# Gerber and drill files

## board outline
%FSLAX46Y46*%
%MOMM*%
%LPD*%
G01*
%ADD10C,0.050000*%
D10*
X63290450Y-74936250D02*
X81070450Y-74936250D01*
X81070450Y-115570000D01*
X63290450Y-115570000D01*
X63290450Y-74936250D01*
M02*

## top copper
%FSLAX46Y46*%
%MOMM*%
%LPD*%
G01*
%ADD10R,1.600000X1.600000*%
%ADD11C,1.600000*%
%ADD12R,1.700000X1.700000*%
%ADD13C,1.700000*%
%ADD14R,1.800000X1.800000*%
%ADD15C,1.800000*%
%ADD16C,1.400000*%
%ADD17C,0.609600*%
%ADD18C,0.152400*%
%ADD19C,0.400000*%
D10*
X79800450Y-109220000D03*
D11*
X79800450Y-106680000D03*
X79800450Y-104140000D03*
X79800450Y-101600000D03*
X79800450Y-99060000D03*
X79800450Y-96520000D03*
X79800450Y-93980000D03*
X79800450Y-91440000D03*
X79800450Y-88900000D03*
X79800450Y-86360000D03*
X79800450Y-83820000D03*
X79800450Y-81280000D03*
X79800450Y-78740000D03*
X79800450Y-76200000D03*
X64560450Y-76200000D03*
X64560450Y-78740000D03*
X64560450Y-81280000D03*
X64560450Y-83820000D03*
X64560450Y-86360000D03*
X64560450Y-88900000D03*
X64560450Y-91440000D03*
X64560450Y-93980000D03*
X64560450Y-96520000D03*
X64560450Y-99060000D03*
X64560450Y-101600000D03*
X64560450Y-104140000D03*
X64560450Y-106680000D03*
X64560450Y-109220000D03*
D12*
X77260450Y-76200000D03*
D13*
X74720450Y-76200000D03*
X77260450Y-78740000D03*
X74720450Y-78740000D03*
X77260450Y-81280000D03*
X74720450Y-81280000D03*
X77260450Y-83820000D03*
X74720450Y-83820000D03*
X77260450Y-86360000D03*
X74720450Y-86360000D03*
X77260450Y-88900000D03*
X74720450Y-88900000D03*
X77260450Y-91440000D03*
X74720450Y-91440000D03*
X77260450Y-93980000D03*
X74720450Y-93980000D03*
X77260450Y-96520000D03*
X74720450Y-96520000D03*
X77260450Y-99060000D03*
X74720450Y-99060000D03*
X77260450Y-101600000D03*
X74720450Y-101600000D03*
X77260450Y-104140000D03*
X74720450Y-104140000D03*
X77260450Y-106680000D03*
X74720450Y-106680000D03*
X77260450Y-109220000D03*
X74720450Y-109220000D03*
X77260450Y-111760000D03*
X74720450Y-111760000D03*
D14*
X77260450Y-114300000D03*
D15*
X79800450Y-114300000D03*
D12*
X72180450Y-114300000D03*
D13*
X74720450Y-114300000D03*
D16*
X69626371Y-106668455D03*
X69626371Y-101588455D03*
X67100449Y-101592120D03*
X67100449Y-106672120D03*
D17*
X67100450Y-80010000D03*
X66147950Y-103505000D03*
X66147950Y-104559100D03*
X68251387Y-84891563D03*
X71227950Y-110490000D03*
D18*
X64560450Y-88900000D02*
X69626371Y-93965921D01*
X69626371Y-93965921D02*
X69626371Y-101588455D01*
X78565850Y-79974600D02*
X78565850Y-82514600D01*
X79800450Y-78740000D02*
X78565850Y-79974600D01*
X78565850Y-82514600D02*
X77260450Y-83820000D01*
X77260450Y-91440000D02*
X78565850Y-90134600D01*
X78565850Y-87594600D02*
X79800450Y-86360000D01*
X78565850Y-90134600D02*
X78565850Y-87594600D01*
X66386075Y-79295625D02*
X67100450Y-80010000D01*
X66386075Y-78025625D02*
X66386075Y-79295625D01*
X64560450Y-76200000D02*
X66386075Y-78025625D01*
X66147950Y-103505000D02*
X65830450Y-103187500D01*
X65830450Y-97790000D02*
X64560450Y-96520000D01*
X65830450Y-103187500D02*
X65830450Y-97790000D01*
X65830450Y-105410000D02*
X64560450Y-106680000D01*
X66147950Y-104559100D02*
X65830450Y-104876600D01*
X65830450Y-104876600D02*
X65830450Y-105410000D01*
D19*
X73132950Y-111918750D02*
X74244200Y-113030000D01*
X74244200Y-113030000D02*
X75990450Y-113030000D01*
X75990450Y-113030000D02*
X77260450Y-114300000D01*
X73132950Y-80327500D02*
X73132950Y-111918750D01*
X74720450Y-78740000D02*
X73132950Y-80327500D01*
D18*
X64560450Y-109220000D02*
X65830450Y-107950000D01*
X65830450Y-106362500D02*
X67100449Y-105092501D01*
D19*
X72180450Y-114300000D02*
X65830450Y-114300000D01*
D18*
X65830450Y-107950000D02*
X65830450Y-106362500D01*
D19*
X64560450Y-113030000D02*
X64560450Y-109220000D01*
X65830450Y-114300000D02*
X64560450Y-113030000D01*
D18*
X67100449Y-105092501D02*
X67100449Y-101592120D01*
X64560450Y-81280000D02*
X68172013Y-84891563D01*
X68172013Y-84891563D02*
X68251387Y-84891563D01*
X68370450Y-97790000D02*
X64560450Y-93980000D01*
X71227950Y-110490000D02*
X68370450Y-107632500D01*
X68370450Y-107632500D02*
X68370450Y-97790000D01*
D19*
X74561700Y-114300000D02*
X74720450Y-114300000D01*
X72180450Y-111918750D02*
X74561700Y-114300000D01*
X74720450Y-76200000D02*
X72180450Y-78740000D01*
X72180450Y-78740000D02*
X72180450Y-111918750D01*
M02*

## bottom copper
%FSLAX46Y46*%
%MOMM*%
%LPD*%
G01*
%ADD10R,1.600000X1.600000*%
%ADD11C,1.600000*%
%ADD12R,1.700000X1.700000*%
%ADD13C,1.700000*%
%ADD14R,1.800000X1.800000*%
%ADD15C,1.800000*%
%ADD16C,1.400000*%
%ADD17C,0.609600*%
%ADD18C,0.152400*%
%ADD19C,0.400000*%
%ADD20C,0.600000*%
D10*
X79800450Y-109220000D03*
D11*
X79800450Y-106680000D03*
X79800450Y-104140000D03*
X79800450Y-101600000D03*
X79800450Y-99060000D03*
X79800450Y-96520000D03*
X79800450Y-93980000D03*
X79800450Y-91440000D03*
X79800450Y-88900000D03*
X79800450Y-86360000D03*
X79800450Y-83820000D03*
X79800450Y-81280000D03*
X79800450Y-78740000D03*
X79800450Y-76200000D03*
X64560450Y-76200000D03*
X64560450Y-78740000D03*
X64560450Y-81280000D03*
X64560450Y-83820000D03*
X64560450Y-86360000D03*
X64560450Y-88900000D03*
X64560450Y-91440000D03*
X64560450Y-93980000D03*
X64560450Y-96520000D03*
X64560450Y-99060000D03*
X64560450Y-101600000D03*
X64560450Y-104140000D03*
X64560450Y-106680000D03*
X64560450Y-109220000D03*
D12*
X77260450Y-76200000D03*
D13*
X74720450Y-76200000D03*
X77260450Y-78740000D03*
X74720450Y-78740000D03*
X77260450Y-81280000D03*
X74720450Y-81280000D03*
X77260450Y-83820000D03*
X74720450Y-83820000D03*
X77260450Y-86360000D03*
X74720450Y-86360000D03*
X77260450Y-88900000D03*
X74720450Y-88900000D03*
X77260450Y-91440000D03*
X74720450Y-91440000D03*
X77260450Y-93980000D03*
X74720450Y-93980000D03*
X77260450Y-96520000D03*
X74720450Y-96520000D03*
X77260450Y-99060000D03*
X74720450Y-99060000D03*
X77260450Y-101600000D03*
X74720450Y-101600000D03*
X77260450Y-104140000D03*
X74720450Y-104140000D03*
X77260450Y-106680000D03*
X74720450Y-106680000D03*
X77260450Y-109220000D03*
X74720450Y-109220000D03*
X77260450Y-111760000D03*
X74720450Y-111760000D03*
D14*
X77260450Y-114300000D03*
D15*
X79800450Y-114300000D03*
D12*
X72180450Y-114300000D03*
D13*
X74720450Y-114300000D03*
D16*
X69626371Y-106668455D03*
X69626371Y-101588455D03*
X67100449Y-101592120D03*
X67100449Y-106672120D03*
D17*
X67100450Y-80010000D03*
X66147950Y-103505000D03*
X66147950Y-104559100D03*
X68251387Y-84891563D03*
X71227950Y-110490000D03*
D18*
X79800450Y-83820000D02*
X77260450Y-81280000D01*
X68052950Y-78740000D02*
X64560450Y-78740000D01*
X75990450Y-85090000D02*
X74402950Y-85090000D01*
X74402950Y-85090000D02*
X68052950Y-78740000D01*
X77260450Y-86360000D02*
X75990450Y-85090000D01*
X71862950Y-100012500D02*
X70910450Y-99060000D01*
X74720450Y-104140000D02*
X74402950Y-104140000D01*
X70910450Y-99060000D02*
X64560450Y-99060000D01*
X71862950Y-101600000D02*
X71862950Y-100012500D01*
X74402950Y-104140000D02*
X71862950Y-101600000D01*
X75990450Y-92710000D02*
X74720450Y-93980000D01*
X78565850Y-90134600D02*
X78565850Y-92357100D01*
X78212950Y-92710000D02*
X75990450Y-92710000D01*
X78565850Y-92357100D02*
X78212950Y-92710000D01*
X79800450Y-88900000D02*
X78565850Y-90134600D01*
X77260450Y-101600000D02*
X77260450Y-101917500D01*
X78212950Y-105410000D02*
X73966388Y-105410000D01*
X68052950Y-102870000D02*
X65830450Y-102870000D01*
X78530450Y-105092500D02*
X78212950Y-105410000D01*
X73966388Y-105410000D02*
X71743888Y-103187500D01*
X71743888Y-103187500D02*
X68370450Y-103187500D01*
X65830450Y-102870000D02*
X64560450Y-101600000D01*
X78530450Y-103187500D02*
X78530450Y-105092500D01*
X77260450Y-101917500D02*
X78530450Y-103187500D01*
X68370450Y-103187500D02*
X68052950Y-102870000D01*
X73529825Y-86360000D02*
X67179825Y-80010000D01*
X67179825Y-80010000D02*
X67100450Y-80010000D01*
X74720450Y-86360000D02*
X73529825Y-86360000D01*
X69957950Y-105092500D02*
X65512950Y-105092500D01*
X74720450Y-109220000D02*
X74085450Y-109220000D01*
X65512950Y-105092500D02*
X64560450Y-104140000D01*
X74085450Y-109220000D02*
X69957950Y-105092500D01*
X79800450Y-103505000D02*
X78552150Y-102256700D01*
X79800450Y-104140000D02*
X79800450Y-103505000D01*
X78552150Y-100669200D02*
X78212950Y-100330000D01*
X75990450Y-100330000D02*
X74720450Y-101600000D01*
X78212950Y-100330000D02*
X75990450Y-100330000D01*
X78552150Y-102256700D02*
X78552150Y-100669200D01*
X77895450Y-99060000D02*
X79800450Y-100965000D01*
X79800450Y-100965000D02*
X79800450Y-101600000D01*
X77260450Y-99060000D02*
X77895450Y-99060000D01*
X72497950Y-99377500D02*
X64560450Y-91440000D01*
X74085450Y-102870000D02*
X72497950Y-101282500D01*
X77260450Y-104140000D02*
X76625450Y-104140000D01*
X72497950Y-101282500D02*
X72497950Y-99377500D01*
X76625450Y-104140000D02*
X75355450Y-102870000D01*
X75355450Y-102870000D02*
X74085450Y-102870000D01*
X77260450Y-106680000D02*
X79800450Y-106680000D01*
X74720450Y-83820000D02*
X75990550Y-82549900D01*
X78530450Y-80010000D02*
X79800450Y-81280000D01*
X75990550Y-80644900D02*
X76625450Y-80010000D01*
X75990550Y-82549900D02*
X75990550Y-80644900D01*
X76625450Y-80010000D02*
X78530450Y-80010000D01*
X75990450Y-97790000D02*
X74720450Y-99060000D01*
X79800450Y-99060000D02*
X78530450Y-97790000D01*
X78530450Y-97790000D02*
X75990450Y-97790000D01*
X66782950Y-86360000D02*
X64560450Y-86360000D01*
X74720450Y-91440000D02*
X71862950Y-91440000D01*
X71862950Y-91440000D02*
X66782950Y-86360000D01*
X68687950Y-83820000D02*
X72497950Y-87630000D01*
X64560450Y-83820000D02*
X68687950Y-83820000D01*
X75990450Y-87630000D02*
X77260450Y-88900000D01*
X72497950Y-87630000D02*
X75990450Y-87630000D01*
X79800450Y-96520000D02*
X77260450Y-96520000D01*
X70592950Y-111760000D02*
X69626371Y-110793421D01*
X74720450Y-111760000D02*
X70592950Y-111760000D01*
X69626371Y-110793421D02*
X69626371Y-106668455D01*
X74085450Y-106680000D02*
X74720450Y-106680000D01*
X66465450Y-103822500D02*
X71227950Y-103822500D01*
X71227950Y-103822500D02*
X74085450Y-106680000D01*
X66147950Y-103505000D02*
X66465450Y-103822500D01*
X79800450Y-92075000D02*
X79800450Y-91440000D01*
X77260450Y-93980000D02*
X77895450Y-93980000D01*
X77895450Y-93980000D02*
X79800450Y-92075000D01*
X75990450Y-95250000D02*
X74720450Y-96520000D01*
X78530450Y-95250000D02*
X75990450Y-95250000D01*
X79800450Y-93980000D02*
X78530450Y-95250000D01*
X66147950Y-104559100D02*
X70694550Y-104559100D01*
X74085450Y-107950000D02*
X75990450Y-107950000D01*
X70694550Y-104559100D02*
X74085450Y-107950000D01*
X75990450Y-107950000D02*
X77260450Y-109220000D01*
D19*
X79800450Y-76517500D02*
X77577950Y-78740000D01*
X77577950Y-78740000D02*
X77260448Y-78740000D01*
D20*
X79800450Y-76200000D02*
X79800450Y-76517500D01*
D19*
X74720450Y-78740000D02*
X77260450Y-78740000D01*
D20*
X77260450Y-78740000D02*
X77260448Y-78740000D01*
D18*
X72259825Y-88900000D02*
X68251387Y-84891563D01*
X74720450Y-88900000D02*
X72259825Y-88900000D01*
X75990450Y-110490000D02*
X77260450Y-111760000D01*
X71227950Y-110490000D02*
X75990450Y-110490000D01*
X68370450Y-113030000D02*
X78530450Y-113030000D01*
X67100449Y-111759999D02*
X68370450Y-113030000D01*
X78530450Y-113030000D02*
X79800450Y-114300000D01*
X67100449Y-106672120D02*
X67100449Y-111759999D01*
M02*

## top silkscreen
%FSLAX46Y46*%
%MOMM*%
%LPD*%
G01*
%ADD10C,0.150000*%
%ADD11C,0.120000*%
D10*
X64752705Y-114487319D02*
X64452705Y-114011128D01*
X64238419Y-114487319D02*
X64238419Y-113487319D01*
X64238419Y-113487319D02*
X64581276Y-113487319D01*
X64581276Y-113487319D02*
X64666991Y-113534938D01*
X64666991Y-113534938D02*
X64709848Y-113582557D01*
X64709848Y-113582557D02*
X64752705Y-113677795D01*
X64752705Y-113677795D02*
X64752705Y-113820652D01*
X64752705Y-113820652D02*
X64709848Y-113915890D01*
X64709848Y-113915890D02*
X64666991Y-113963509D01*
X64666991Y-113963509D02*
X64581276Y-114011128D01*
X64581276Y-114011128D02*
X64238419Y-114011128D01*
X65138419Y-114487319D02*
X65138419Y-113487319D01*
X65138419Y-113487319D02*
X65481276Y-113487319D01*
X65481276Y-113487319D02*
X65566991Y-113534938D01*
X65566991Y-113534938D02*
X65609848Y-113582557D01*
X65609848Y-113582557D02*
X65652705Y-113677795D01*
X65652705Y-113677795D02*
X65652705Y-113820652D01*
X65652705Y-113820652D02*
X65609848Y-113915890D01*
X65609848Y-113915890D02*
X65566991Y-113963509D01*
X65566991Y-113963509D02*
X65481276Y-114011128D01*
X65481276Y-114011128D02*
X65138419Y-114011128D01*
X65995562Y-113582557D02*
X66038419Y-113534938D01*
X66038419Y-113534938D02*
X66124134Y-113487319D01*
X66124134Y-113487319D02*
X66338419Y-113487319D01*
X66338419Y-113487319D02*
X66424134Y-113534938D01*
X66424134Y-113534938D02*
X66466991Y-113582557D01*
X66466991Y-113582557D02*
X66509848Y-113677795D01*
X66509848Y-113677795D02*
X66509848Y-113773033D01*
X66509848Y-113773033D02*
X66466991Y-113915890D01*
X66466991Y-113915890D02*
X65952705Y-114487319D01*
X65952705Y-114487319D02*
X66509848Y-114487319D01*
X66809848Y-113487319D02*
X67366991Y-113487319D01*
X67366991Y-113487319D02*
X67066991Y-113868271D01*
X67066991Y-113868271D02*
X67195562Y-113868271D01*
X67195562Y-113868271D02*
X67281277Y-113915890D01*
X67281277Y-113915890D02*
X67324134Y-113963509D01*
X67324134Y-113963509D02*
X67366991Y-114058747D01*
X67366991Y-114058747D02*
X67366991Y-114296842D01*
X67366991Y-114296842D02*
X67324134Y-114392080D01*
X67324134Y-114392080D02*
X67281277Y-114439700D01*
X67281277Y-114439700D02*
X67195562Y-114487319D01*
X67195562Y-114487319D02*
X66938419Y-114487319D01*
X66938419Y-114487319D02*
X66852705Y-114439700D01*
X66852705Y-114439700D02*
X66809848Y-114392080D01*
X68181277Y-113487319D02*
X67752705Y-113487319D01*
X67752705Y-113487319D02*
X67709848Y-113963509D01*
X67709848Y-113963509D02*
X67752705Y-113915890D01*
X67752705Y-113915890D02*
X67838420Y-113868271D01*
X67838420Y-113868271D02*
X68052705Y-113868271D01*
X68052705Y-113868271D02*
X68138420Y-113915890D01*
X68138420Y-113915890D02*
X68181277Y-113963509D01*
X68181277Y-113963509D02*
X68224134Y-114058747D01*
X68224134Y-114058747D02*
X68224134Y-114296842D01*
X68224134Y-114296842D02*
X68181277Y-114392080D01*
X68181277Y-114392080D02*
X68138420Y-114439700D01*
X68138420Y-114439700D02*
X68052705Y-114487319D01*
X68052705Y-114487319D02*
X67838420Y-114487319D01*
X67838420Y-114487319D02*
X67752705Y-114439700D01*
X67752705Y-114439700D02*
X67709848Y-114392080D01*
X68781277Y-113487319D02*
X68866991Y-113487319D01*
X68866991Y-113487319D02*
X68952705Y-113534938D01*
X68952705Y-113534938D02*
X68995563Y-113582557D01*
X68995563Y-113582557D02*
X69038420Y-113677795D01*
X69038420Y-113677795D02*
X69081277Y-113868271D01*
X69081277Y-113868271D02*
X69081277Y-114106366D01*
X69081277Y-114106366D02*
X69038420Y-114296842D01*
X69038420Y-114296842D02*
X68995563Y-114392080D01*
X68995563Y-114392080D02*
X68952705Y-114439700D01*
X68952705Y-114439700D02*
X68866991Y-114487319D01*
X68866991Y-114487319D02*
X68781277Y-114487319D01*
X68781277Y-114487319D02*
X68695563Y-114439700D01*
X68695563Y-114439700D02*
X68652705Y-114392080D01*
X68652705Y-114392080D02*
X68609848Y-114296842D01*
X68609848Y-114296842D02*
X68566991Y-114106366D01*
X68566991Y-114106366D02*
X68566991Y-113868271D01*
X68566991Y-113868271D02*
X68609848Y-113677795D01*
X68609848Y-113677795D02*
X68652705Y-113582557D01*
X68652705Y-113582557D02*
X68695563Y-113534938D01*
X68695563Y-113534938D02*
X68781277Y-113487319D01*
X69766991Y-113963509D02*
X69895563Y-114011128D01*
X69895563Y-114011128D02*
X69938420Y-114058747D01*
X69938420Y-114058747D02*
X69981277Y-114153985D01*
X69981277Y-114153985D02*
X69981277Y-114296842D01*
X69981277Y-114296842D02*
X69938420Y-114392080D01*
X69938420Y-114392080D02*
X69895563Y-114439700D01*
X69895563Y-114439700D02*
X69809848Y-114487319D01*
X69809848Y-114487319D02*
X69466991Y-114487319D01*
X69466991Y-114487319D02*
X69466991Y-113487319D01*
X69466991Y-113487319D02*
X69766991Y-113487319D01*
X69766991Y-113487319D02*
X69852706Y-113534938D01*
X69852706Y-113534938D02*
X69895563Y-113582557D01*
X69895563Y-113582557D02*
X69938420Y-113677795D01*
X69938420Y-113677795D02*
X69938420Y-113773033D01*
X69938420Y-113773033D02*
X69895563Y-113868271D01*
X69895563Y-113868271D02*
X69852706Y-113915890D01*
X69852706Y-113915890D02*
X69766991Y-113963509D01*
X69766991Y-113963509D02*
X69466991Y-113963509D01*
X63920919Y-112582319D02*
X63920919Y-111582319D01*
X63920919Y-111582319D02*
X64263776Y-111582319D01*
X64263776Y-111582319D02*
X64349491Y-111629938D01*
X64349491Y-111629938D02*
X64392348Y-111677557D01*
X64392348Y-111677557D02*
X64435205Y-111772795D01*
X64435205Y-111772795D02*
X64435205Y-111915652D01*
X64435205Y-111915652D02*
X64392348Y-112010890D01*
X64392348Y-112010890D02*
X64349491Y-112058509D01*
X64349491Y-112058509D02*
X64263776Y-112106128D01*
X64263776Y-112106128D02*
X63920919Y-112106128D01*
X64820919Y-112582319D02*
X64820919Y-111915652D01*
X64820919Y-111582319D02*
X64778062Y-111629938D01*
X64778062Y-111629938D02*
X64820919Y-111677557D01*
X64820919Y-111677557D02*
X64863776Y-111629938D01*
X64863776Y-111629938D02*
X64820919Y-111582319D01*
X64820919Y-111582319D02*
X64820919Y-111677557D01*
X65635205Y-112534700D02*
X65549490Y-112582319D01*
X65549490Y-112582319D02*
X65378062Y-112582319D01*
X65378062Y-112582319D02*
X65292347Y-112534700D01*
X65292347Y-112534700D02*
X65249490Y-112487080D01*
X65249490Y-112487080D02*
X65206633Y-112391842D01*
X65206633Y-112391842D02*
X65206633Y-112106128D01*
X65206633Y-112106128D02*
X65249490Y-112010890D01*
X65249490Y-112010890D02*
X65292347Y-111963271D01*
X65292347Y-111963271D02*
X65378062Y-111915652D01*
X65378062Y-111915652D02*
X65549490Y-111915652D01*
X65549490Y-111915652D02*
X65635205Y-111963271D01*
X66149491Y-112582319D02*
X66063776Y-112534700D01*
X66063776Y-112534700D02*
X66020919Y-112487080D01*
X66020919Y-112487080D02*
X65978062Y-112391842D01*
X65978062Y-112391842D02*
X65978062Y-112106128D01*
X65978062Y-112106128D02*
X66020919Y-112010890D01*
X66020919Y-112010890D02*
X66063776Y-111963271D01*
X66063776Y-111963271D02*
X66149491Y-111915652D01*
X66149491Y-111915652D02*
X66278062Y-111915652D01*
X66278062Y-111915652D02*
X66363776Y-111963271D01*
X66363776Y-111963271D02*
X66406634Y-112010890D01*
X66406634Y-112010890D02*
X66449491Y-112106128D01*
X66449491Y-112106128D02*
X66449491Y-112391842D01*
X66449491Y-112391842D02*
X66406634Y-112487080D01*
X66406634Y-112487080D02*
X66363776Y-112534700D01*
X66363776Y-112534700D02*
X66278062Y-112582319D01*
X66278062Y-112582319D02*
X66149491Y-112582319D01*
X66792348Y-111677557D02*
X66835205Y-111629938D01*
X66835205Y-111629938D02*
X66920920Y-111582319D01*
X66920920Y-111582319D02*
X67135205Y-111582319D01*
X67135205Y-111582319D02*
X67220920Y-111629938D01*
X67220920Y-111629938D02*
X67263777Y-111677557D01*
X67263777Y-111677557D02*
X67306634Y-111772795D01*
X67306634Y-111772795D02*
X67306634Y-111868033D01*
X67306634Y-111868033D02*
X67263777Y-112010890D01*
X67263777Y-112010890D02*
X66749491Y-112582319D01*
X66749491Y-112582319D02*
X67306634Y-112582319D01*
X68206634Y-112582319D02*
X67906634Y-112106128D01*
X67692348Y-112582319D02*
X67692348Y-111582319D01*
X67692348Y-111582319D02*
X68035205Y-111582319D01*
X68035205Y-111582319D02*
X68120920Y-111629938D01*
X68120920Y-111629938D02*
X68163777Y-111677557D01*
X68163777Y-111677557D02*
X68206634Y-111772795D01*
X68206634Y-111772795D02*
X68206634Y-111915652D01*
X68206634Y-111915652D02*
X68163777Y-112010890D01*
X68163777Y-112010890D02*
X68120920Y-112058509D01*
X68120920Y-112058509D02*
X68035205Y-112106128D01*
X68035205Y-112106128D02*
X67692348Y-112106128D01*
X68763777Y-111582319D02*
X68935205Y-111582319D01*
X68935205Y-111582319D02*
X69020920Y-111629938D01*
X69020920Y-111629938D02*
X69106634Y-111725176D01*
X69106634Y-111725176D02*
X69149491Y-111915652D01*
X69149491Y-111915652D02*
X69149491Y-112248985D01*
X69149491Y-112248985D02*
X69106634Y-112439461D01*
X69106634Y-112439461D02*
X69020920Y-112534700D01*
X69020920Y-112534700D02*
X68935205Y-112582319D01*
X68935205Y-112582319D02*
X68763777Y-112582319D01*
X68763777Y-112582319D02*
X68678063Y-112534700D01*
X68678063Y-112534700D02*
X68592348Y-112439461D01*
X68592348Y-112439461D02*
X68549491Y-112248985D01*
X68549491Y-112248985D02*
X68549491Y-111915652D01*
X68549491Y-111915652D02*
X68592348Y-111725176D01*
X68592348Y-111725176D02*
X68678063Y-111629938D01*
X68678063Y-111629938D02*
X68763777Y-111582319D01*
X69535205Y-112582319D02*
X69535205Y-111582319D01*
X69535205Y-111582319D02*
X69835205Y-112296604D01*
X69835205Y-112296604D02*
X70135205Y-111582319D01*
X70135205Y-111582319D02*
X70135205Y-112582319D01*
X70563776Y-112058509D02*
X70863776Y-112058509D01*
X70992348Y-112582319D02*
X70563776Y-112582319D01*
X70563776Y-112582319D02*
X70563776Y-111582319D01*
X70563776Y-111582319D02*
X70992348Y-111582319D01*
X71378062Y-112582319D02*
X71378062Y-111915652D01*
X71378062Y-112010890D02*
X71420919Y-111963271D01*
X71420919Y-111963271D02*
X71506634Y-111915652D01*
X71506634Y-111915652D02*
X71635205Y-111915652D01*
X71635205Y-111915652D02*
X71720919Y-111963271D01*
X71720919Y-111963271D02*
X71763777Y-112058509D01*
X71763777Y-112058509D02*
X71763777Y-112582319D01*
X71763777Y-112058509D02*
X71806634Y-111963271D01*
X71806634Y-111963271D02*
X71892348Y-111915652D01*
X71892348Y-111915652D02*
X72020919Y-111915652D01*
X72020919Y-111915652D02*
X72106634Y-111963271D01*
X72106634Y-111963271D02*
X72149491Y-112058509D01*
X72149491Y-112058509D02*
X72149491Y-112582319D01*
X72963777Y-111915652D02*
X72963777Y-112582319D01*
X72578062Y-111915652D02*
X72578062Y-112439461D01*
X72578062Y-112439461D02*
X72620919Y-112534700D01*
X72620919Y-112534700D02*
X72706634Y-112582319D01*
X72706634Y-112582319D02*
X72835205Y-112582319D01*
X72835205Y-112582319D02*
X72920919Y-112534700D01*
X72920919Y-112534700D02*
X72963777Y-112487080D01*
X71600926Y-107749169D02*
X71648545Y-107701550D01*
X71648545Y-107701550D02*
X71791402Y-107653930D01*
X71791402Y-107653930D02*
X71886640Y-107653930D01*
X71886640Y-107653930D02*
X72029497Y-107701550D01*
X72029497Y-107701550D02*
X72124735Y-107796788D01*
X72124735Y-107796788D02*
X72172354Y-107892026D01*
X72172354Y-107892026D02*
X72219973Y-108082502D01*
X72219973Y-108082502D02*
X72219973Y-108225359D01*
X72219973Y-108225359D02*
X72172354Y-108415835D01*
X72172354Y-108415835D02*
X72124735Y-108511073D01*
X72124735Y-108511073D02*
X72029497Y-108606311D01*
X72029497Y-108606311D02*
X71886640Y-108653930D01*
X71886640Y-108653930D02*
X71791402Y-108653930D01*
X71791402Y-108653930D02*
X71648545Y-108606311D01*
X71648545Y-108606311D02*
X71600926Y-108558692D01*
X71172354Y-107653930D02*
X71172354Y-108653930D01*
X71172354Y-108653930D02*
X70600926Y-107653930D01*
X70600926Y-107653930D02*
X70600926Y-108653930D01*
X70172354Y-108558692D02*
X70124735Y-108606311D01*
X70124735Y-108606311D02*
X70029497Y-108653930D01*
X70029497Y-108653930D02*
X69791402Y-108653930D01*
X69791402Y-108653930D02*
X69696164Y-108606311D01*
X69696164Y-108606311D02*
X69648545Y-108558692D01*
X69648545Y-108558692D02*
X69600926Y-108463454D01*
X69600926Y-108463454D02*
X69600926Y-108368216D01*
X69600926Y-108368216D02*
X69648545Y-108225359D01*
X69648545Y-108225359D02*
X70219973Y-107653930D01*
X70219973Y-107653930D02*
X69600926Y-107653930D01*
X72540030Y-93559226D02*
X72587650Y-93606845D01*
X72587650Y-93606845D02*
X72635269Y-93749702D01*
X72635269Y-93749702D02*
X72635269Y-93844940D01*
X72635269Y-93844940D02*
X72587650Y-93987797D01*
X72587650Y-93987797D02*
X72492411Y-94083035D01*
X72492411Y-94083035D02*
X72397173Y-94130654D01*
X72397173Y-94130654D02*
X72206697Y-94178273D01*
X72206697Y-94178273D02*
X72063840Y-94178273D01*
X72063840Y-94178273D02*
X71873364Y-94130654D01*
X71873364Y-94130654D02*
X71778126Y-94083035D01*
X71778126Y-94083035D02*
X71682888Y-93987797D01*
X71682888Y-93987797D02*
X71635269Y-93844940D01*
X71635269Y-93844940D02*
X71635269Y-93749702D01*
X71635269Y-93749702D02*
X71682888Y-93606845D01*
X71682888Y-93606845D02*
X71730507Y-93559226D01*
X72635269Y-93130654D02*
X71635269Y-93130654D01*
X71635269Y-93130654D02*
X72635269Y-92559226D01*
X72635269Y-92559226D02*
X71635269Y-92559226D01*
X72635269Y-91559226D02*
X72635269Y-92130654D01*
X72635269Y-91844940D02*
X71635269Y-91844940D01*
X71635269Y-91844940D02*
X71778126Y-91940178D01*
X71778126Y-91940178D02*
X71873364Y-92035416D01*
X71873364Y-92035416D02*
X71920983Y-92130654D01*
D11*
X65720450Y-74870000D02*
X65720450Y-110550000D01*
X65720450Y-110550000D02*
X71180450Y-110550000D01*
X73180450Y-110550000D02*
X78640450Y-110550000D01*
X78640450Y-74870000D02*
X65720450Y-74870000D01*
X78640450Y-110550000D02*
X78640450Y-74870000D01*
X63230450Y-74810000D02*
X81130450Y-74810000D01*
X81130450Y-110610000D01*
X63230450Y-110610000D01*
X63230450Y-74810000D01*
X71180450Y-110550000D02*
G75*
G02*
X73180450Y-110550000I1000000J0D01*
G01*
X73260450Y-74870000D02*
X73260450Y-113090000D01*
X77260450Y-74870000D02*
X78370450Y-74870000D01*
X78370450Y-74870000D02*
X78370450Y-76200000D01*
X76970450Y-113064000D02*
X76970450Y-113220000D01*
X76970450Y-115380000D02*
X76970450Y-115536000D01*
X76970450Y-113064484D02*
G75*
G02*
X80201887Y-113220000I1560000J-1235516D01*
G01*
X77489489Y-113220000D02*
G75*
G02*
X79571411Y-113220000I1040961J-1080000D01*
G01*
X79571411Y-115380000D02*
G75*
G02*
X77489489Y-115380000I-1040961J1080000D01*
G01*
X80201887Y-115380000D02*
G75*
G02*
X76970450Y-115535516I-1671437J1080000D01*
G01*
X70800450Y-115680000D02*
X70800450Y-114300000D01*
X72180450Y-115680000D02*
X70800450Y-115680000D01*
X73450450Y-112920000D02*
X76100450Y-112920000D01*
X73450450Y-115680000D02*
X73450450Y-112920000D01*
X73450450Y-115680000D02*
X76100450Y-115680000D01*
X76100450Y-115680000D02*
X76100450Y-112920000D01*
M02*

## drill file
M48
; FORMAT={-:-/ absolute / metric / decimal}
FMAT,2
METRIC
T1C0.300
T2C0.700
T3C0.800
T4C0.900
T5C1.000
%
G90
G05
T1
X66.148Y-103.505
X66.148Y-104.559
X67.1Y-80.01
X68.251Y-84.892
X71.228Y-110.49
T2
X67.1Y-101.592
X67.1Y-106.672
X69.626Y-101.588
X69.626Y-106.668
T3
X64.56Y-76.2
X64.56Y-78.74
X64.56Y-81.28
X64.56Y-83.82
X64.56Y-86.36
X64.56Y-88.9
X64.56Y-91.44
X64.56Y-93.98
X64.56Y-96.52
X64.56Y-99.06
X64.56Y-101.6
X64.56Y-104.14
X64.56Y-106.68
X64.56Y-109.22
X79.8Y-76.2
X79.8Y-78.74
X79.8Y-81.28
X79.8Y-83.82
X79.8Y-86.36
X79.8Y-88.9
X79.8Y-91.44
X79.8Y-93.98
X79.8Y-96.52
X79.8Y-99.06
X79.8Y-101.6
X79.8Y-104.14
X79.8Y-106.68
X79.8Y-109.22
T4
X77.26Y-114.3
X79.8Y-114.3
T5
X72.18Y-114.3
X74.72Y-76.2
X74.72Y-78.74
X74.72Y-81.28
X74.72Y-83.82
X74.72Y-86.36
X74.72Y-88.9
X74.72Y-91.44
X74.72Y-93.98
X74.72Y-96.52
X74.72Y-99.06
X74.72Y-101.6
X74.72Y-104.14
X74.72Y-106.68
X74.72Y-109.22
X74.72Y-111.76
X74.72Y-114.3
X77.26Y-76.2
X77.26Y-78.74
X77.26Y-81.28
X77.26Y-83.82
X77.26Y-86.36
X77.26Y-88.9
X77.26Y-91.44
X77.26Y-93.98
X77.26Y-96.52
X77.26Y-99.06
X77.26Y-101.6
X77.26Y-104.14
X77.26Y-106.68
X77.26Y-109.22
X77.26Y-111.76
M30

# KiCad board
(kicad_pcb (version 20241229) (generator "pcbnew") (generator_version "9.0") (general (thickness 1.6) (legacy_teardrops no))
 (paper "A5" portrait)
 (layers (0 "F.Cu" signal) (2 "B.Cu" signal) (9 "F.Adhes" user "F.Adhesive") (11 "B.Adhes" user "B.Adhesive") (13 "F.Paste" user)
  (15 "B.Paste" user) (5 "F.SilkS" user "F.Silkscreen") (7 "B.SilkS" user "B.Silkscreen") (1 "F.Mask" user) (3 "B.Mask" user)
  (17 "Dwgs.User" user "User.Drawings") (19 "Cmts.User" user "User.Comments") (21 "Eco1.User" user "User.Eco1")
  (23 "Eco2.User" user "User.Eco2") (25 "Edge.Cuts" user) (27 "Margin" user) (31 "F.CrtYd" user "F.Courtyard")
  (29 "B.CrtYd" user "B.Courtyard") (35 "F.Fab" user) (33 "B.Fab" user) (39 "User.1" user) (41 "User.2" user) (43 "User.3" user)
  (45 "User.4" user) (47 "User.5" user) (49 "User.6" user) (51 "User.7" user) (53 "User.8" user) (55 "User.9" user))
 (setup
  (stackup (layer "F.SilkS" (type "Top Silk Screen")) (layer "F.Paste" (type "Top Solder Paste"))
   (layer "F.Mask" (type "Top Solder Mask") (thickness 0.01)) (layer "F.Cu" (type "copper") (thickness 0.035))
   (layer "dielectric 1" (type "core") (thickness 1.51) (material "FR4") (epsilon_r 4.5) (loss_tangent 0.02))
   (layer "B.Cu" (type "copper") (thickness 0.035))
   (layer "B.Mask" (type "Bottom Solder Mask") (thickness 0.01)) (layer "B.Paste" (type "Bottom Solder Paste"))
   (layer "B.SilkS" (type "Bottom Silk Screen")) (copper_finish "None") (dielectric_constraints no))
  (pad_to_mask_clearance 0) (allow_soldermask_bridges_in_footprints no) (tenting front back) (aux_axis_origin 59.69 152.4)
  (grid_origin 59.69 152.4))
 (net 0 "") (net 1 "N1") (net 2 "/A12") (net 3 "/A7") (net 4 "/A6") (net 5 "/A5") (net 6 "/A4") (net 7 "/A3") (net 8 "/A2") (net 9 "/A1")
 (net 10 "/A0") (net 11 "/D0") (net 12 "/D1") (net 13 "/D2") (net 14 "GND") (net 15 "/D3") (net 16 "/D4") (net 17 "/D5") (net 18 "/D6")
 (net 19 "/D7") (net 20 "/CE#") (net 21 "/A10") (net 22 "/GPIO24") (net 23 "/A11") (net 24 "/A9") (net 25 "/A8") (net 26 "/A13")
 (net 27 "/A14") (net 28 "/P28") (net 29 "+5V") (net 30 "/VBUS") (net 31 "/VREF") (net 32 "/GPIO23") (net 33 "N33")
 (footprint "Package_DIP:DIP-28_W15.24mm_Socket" (layer "F.Cu") (at 79.80045 109.22 180)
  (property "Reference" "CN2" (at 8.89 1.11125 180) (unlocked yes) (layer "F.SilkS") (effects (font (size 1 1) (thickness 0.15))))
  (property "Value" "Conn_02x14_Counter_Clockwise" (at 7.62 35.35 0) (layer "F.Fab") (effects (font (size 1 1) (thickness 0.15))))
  (fp_line (start 14.08 34.35) (end 14.08 -1.33) (stroke (width 0.12) (type solid)) (layer "F.SilkS"))
  (fp_line (start 14.08 -1.33) (end 8.62 -1.33) (stroke (width 0.12) (type solid)) (layer "F.SilkS"))
  (fp_line (start 6.62 -1.33) (end 1.16 -1.33) (stroke (width 0.12) (type solid)) (layer "F.SilkS"))
  (fp_line (start 1.16 34.35) (end 14.08 34.35) (stroke (width 0.12) (type solid)) (layer "F.SilkS"))
  (fp_line (start 1.16 -1.33) (end 1.16 34.35) (stroke (width 0.12) (type solid)) (layer "F.SilkS"))
  (fp_rect (start -1.33 -1.39) (end 16.57 34.41) (stroke (width 0.12) (type solid)) (fill no) (layer "F.SilkS"))
  (fp_arc (start 8.62 -1.33) (mid 7.62 -0.33) (end 6.62 -1.33) (stroke (width 0.12) (type solid)) (layer "F.SilkS"))
  (pad "1" thru_hole rect (at 0 0 180) (size 1.6 1.6) (drill 0.8) (layers "*.Cu" "*.Mask") (remove_unused_layers no) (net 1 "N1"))
  (pad "2" thru_hole circle (at 0 2.54 180) (size 1.6 1.6) (drill 0.8) (layers "*.Cu" "*.Mask") (remove_unused_layers no) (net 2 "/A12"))
  (pad "3" thru_hole circle (at 0 5.08 180) (size 1.6 1.6) (drill 0.8) (layers "*.Cu" "*.Mask") (remove_unused_layers no) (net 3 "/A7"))
  (pad "4" thru_hole circle (at 0 7.62 180) (size 1.6 1.6) (drill 0.8) (layers "*.Cu" "*.Mask") (remove_unused_layers no) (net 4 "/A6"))
  (pad "5" thru_hole circle (at 0 10.16 180) (size 1.6 1.6) (drill 0.8) (layers "*.Cu" "*.Mask") (remove_unused_layers no) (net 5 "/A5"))
  (pad "6" thru_hole circle (at 0 12.7 180) (size 1.6 1.6) (drill 0.8) (layers "*.Cu" "*.Mask") (remove_unused_layers no) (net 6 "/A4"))
  (pad "7" thru_hole circle (at 0 15.24 180) (size 1.6 1.6) (drill 0.8) (layers "*.Cu" "*.Mask") (remove_unused_layers no) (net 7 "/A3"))
  (pad "8" thru_hole circle (at 0 17.78 180) (size 1.6 1.6) (drill 0.8) (layers "*.Cu" "*.Mask") (remove_unused_layers no) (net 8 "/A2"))
  (pad "9" thru_hole circle (at 0 20.32 180) (size 1.6 1.6) (drill 0.8) (layers "*.Cu" "*.Mask") (remove_unused_layers no) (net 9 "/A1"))
  (pad "10" thru_hole circle (at 0 22.86 180) (size 1.6 1.6) (drill 0.8) (layers "*.Cu" "*.Mask") (remove_unused_layers no) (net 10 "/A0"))
  (pad "11" thru_hole circle (at 0 25.4 180) (size 1.6 1.6) (drill 0.8) (layers "*.Cu" "*.Mask") (remove_unused_layers no) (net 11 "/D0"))
  (pad "12" thru_hole circle (at 0 27.94 180) (size 1.6 1.6) (drill 0.8) (layers "*.Cu" "*.Mask") (remove_unused_layers no) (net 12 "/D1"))
  (pad "13" thru_hole circle (at 0 30.48 180) (size 1.6 1.6) (drill 0.8) (layers "*.Cu" "*.Mask") (remove_unused_layers no) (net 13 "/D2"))
  (pad "14" thru_hole circle (at 0 33.02 180) (size 1.6 1.6) (drill 0.8) (layers "*.Cu" "*.Mask") (remove_unused_layers no) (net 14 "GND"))
  (pad "15" thru_hole circle (at 15.24 33.02 180) (size 1.6 1.6) (drill 0.8) (layers "*.Cu" "*.Mask") (remove_unused_layers no)
   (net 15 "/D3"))
  (pad "16" thru_hole circle (at 15.24 30.48 180) (size 1.6 1.6) (drill 0.8) (layers "*.Cu" "*.Mask") (remove_unused_layers no)
   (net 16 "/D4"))
  (pad "17" thru_hole circle (at 15.24 27.94 180) (size 1.6 1.6) (drill 0.8) (layers "*.Cu" "*.Mask") (remove_unused_layers no)
   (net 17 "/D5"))
  (pad "18" thru_hole circle (at 15.24 25.4 180) (size 1.6 1.6) (drill 0.8) (layers "*.Cu" "*.Mask") (remove_unused_layers no)
   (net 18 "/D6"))
  (pad "19" thru_hole circle (at 15.24 22.86 180) (size 1.6 1.6) (drill 0.8) (layers "*.Cu" "*.Mask") (remove_unused_layers no)
   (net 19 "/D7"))
  (pad "20" thru_hole circle (at 15.24 20.32 180) (size 1.6 1.6) (drill 0.8) (layers "*.Cu" "*.Mask") (remove_unused_layers no)
   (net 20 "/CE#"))
  (pad "21" thru_hole circle (at 15.24 17.78 180) (size 1.6 1.6) (drill 0.8) (layers "*.Cu" "*.Mask") (remove_unused_layers no)
   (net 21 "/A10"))
  (pad "22" thru_hole circle (at 15.24 15.24 180) (size 1.6 1.6) (drill 0.8) (layers "*.Cu" "*.Mask") (remove_unused_layers no)
   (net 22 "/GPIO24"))
  (pad "23" thru_hole circle (at 15.24 12.7 180) (size 1.6 1.6) (drill 0.8) (layers "*.Cu" "*.Mask") (remove_unused_layers no)
   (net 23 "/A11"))
  (pad "24" thru_hole circle (at 15.24 10.16 180) (size 1.6 1.6) (drill 0.8) (layers "*.Cu" "*.Mask") (remove_unused_layers no)
   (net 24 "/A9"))
  (pad "25" thru_hole circle (at 15.24 7.62 180) (size 1.6 1.6) (drill 0.8) (layers "*.Cu" "*.Mask") (remove_unused_layers no)
   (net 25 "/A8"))
  (pad "26" thru_hole circle (at 15.24 5.08 180) (size 1.6 1.6) (drill 0.8) (layers "*.Cu" "*.Mask") (remove_unused_layers no)
   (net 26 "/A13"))
  (pad "27" thru_hole circle (at 15.24 2.54 180) (size 1.6 1.6) (drill 0.8) (layers "*.Cu" "*.Mask") (remove_unused_layers no)
   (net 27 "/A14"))
  (pad "28" thru_hole circle (at 15.24 0 180) (size 1.6 1.6) (drill 0.8) (layers "*.Cu" "*.Mask") (remove_unused_layers no) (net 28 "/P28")))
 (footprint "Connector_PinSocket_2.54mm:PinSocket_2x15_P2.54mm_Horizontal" (layer "F.Cu") (at 77.26045 76.2)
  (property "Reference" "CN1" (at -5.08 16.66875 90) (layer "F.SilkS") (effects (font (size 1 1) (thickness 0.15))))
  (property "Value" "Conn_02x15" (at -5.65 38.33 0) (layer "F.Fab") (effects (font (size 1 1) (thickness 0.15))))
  (fp_line (start -4 -1.33) (end -4 36.89) (stroke (width 0.12) (type solid)) (layer "F.SilkS"))
  (fp_line (start 0 -1.33) (end 1.11 -1.33) (stroke (width 0.12) (type solid)) (layer "F.SilkS"))
  (fp_line (start 1.11 -1.33) (end 1.11 0) (stroke (width 0.12) (type solid)) (layer "F.SilkS"))
  (pad "1" thru_hole rect (at 0 0) (size 1.7 1.7) (drill 1) (layers "*.Cu" "*.Mask") (remove_unused_layers no) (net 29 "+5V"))
  (pad "2" thru_hole circle (at -2.54 0) (size 1.7 1.7) (drill 1) (layers "*.Cu" "*.Mask") (remove_unused_layers no) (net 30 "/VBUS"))
  (pad "3" thru_hole circle (at 0 2.54) (size 1.7 1.7) (drill 1) (layers "*.Cu" "*.Mask") (remove_unused_layers no) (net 14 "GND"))
  (pad "4" thru_hole circle (at -2.54 2.54) (size 1.7 1.7) (drill 1) (layers "*.Cu" "*.Mask") (remove_unused_layers no) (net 14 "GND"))
  (pad "5" thru_hole circle (at 0 5.08) (size 1.7 1.7) (drill 1) (layers "*.Cu" "*.Mask") (remove_unused_layers no) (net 11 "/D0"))
  (pad "6" thru_hole circle (at -2.54 5.08) (size 1.7 1.7) (drill 1) (layers "*.Cu" "*.Mask") (remove_unused_layers no) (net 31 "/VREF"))
  (pad "7" thru_hole circle (at 0 7.62) (size 1.7 1.7) (drill 1) (layers "*.Cu" "*.Mask") (remove_unused_layers no) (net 13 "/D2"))
  (pad "8" thru_hole circle (at -2.54 7.62) (size 1.7 1.7) (drill 1) (layers "*.Cu" "*.Mask") (remove_unused_layers no) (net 12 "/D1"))
  (pad "9" thru_hole circle (at 0 10.16) (size 1.7 1.7) (drill 1) (layers "*.Cu" "*.Mask") (remove_unused_layers no) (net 16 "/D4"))
  (pad "10" thru_hole circle (at -2.54 10.16) (size 1.7 1.7) (drill 1) (layers "*.Cu" "*.Mask") (remove_unused_layers no) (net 15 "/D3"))
  (pad "11" thru_hole circle (at 0 12.7) (size 1.7 1.7) (drill 1) (layers "*.Cu" "*.Mask") (remove_unused_layers no) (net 18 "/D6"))
  (pad "12" thru_hole circle (at -2.54 12.7) (size 1.7 1.7) (drill 1) (layers "*.Cu" "*.Mask") (remove_unused_layers no) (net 17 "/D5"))
  (pad "13" thru_hole circle (at 0 15.24) (size 1.7 1.7) (drill 1) (layers "*.Cu" "*.Mask") (remove_unused_layers no) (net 10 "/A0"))
  (pad "14" thru_hole circle (at -2.54 15.24) (size 1.7 1.7) (drill 1) (layers "*.Cu" "*.Mask") (remove_unused_layers no) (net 19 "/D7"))
  (pad "15" thru_hole circle (at 0 17.78) (size 1.7 1.7) (drill 1) (layers "*.Cu" "*.Mask") (remove_unused_layers no) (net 8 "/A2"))
  (pad "16" thru_hole circle (at -2.54 17.78) (size 1.7 1.7) (drill 1) (layers "*.Cu" "*.Mask") (remove_unused_layers no) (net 9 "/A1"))
  (pad "17" thru_hole circle (at 0 20.32) (size 1.7 1.7) (drill 1) (layers "*.Cu" "*.Mask") (remove_unused_layers no) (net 6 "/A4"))
  (pad "18" thru_hole circle (at -2.54 20.32) (size 1.7 1.7) (drill 1) (layers "*.Cu" "*.Mask") (remove_unused_layers no) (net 7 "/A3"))
  (pad "19" thru_hole circle (at 0 22.86) (size 1.7 1.7) (drill 1) (layers "*.Cu" "*.Mask") (remove_unused_layers no) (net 4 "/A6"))
  (pad "20" thru_hole circle (at -2.54 22.86) (size 1.7 1.7) (drill 1) (layers "*.Cu" "*.Mask") (remove_unused_layers no) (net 5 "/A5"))
  (pad "21" thru_hole circle (at 0 25.4) (size 1.7 1.7) (drill 1) (layers "*.Cu" "*.Mask") (remove_unused_layers no) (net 25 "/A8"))
  (pad "22" thru_hole circle (at -2.54 25.4) (size 1.7 1.7) (drill 1) (layers "*.Cu" "*.Mask") (remove_unused_layers no) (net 3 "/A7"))
  (pad "23" thru_hole circle (at 0 27.94) (size 1.7 1.7) (drill 1) (layers "*.Cu" "*.Mask") (remove_unused_layers no) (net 21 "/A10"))
  (pad "24" thru_hole circle (at -2.54 27.94) (size 1.7 1.7) (drill 1) (layers "*.Cu" "*.Mask") (remove_unused_layers no) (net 24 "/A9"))
  (pad "25" thru_hole circle (at 0 30.48) (size 1.7 1.7) (drill 1) (layers "*.Cu" "*.Mask") (remove_unused_layers no) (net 2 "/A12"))
  (pad "26" thru_hole circle (at -2.54 30.48) (size 1.7 1.7) (drill 1) (layers "*.Cu" "*.Mask") (remove_unused_layers no) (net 23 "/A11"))
  (pad "27" thru_hole circle (at 0 33.02) (size 1.7 1.7) (drill 1) (layers "*.Cu" "*.Mask") (remove_unused_layers no) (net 27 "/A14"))
  (pad "28" thru_hole circle (at -2.54 33.02) (size 1.7 1.7) (drill 1) (layers "*.Cu" "*.Mask") (remove_unused_layers no) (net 26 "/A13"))
  (pad "29" thru_hole circle (at 0 35.56) (size 1.7 1.7) (drill 1) (layers "*.Cu" "*.Mask") (remove_unused_layers no) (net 22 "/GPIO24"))
  (pad "30" thru_hole circle (at -2.54 35.56) (size 1.7 1.7) (drill 1) (layers "*.Cu" "*.Mask") (remove_unused_layers no) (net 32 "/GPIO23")))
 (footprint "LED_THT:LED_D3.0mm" (layer "F.Cu") (at 77.26045 114.3)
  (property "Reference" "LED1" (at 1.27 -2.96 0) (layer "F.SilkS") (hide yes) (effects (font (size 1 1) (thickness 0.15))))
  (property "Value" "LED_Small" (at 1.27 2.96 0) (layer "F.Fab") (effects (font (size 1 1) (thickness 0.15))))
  (fp_line (start -0.29 -1.236) (end -0.29 -1.08) (stroke (width 0.12) (type solid)) (layer "F.SilkS"))
  (fp_line (start -0.29 1.08) (end -0.29 1.236) (stroke (width 0.12) (type solid)) (layer "F.SilkS"))
  (fp_arc (start -0.29 -1.235516) (mid 1.36566 -1.987699) (end 2.941437 -1.08) (stroke (width 0.12) (type solid)) (layer "F.SilkS"))
  (fp_arc (start 0.229039 -1.08) (mid 1.27 -1.5) (end 2.310961 -1.08) (stroke (width 0.12) (type solid)) (layer "F.SilkS"))
  (fp_arc (start 2.310961 1.08) (mid 1.27 1.5) (end 0.229039 1.08) (stroke (width 0.12) (type solid)) (layer "F.SilkS"))
  (fp_arc (start 2.941437 1.08) (mid 1.36566 1.987699) (end -0.29 1.235516) (stroke (width 0.12) (type solid)) (layer "F.SilkS"))
  (pad "1" thru_hole rect (at 0 0) (size 1.8 1.8) (drill 0.9) (layers "*.Cu" "*.Mask") (remove_unused_layers no) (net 14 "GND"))
  (pad "2" thru_hole circle (at 2.54 0) (size 1.8 1.8) (drill 0.9) (layers "*.Cu" "*.Mask") (remove_unused_layers no) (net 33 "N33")))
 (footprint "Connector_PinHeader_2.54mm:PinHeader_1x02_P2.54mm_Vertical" (layer "F.Cu") (at 72.18045 114.3 90)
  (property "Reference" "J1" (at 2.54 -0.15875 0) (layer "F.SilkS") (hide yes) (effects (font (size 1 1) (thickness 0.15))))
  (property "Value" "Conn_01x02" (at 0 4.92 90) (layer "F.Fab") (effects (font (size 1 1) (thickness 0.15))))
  (fp_line (start -1.38 -1.38) (end 0 -1.38) (stroke (width 0.12) (type solid)) (layer "F.SilkS"))
  (fp_line (start -1.38 0) (end -1.38 -1.38) (stroke (width 0.12) (type solid)) (layer "F.SilkS"))
  (fp_line (start 1.38 1.27) (end 1.38 3.92) (stroke (width 0.12) (type solid)) (layer "F.SilkS"))
  (fp_line (start -1.38 1.27) (end 1.38 1.27) (stroke (width 0.12) (type solid)) (layer "F.SilkS"))
  (fp_line (start -1.38 1.27) (end -1.38 3.92) (stroke (width 0.12) (type solid)) (layer "F.SilkS"))
  (fp_line (start -1.38 3.92) (end 1.38 3.92) (stroke (width 0.12) (type solid)) (layer "F.SilkS"))
  (pad "1" thru_hole rect (at 0 0 90) (size 1.7 1.7) (drill 1) (layers "*.Cu" "*.Mask") (remove_unused_layers no) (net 28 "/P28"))
  (pad "2" thru_hole circle (at 0 2.54 90) (size 1.7 1.7) (drill 1) (layers "*.Cu" "*.Mask") (remove_unused_layers no) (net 30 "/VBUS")))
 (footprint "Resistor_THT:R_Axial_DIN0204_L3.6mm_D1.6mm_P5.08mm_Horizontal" (layer "B.Cu") (at 69.626371 106.668455 90)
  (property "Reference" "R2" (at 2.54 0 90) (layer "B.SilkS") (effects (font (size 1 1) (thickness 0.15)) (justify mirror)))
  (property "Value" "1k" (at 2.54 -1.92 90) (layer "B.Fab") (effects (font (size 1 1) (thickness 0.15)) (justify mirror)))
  (pad "1" thru_hole circle (at 0 0 90) (size 1.4 1.4) (drill 0.7) (layers "*.Cu" "*.Mask") (remove_unused_layers no) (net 32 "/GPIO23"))
  (pad "2" thru_hole circle (at 5.08 0 90) (size 1.4 1.4) (drill 0.7) (layers "*.Cu" "*.Mask") (remove_unused_layers no) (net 20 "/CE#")))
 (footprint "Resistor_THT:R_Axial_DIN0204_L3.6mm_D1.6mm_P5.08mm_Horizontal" (layer "B.Cu") (at 67.100449 101.59212 -90)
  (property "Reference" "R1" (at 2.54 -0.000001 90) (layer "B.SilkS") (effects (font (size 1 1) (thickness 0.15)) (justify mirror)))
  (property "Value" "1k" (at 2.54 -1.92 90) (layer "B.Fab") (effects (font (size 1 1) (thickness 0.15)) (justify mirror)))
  (pad "1" thru_hole circle (at 0 0 270) (size 1.4 1.4) (drill 0.7) (layers "*.Cu" "*.Mask") (remove_unused_layers no) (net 28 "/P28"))
  (pad "2" thru_hole circle (at 5.08 0 270) (size 1.4 1.4) (drill 0.7) (layers "*.Cu" "*.Mask") (remove_unused_layers no) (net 33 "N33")))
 (gr_rect (start 63.29045 74.93625) (end 81.07045 115.57) (stroke (width 0.05) (type default)) (fill no) (layer "Edge.Cuts"))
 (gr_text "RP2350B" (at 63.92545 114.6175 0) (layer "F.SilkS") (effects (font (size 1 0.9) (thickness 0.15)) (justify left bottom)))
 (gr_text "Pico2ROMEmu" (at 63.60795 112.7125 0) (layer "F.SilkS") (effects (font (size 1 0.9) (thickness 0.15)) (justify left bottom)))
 (segment (start 64.56045 88.9) (end 69.626371 93.965921) (width 0.1524) (layer "F.Cu") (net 20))
 (segment (start 69.626371 93.965921) (end 69.626371 101.588455) (width 0.1524) (layer "F.Cu") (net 20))
 (segment (start 79.80045 83.82) (end 77.26045 81.28) (width 0.1524) (layer "B.Cu") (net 11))
 (segment (start 68.05295 78.74) (end 64.56045 78.74) (width 0.1524) (layer "B.Cu") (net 16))
 (segment (start 75.99045 85.09) (end 74.40295 85.09) (width 0.1524) (layer "B.Cu") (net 16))
 (segment (start 74.40295 85.09) (end 68.05295 78.74) (width 0.1524) (layer "B.Cu") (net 16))
 (segment (start 77.26045 86.36) (end 75.99045 85.09) (width 0.1524) (layer "B.Cu") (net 16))
 (segment (start 71.86295 100.0125) (end 70.91045 99.06) (width 0.1524) (layer "B.Cu") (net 24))
 (segment (start 74.72045 104.14) (end 74.40295 104.14) (width 0.1524) (layer "B.Cu") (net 24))
 (segment (start 70.91045 99.06) (end 64.56045 99.06) (width 0.1524) (layer "B.Cu") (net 24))
 (segment (start 71.86295 101.6) (end 71.86295 100.0125) (width 0.1524) (layer "B.Cu") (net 24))
 (segment (start 74.40295 104.14) (end 71.86295 101.6) (width 0.1524) (layer "B.Cu") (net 24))
 (segment (start 78.56585 79.9746) (end 78.56585 82.5146) (width 0.1524) (layer "F.Cu") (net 13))
 (segment (start 79.80045 78.74) (end 78.56585 79.9746) (width 0.1524) (layer "F.Cu") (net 13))
 (segment (start 78.56585 82.5146) (end 77.26045 83.82) (width 0.1524) (layer "F.Cu") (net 13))
 (segment (start 75.99045 92.71) (end 74.72045 93.98) (width 0.1524) (layer "B.Cu") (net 9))
 (segment (start 78.56585 90.1346) (end 78.56585 92.3571) (width 0.1524) (layer "B.Cu") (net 9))
 (segment (start 78.21295 92.71) (end 75.99045 92.71) (width 0.1524) (layer "B.Cu") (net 9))
 (segment (start 78.56585 92.3571) (end 78.21295 92.71) (width 0.1524) (layer "B.Cu") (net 9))
 (segment (start 79.80045 88.9) (end 78.56585 90.1346) (width 0.1524) (layer "B.Cu") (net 9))
 (segment (start 77.26045 101.6) (end 77.26045 101.9175) (width 0.1524) (layer "B.Cu") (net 25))
 (segment (start 78.21295 105.41) (end 73.966388 105.41) (width 0.1524) (layer "B.Cu") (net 25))
 (segment (start 68.05295 102.87) (end 65.83045 102.87) (width 0.1524) (layer "B.Cu") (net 25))
 (segment (start 78.53045 105.0925) (end 78.21295 105.41) (width 0.1524) (layer "B.Cu") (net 25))
 (segment (start 73.966388 105.41) (end 71.743888 103.1875) (width 0.1524) (layer "B.Cu") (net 25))
 (segment (start 71.743888 103.1875) (end 68.37045 103.1875) (width 0.1524) (layer "B.Cu") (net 25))
 (segment (start 65.83045 102.87) (end 64.56045 101.6) (width 0.1524) (layer "B.Cu") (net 25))
 (segment (start 78.53045 103.1875) (end 78.53045 105.0925) (width 0.1524) (layer "B.Cu") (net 25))
 (segment (start 77.26045 101.9175) (end 78.53045 103.1875) (width 0.1524) (layer "B.Cu") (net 25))
 (segment (start 68.37045 103.1875) (end 68.05295 102.87) (width 0.1524) (layer "B.Cu") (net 25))
 (segment (start 77.26045 91.44) (end 78.56585 90.1346) (width 0.1524) (layer "F.Cu") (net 10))
 (segment (start 78.56585 87.5946) (end 79.80045 86.36) (width 0.1524) (layer "F.Cu") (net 10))
 (segment (start 78.56585 90.1346) (end 78.56585 87.5946) (width 0.1524) (layer "F.Cu") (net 10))
 (segment (start 66.386075 79.295625) (end 67.10045 80.01) (width 0.1524) (layer "F.Cu") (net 15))
 (segment (start 66.386075 78.025625) (end 66.386075 79.295625) (width 0.1524) (layer "F.Cu") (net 15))
 (segment (start 64.56045 76.2) (end 66.386075 78.025625) (width 0.1524) (layer "F.Cu") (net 15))
 (via (at 67.10045 80.01) (size 0.6096) (drill 0.3) (layers "F.Cu" "B.Cu") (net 15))
 (segment (start 73.529825 86.36) (end 67.179825 80.01) (width 0.1524) (layer "B.Cu") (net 15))
 (segment (start 67.179825 80.01) (end 67.10045 80.01) (width 0.1524) (layer "B.Cu") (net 15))
 (segment (start 74.72045 86.36) (end 73.529825 86.36) (width 0.1524) (layer "B.Cu") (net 15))
 (segment (start 69.95795 105.0925) (end 65.51295 105.0925) (width 0.1524) (layer "B.Cu") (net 26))
 (segment (start 74.72045 109.22) (end 74.08545 109.22) (width 0.1524) (layer "B.Cu") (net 26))
 (segment (start 65.51295 105.0925) (end 64.56045 104.14) (width 0.1524) (layer "B.Cu") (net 26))
 (segment (start 74.08545 109.22) (end 69.95795 105.0925) (width 0.1524) (layer "B.Cu") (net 26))
 (segment (start 79.80045 103.505) (end 78.55215 102.2567) (width 0.1524) (layer "B.Cu") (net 3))
 (segment (start 79.80045 104.14) (end 79.80045 103.505) (width 0.1524) (layer "B.Cu") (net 3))
 (segment (start 78.55215 100.6692) (end 78.21295 100.33) (width 0.1524) (layer "B.Cu") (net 3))
 (segment (start 75.99045 100.33) (end 74.72045 101.6) (width 0.1524) (layer "B.Cu") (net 3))
 (segment (start 78.21295 100.33) (end 75.99045 100.33) (width 0.1524) (layer "B.Cu") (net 3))
 (segment (start 78.55215 102.2567) (end 78.55215 100.6692) (width 0.1524) (layer "B.Cu") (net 3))
 (segment (start 77.89545 99.06) (end 79.80045 100.965) (width 0.1524) (layer "B.Cu") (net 4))
 (segment (start 79.80045 100.965) (end 79.80045 101.6) (width 0.1524) (layer "B.Cu") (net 4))
 (segment (start 77.26045 99.06) (end 77.89545 99.06) (width 0.1524) (layer "B.Cu") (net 4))
 (segment (start 72.49795 99.3775) (end 64.56045 91.44) (width 0.1524) (layer "B.Cu") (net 21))
 (segment (start 74.08545 102.87) (end 72.49795 101.2825) (width 0.1524) (layer "B.Cu") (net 21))
 (segment (start 77.26045 104.14) (end 76.62545 104.14) (width 0.1524) (layer "B.Cu") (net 21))
 (segment (start 72.49795 101.2825) (end 72.49795 99.3775) (width 0.1524) (layer "B.Cu") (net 21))
 (segment (start 76.62545 104.14) (end 75.35545 102.87) (width 0.1524) (layer "B.Cu") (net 21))
 (segment (start 75.35545 102.87) (end 74.08545 102.87) (width 0.1524) (layer "B.Cu") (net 21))
 (segment (start 77.26045 106.68) (end 79.80045 106.68) (width 0.1524) (layer "B.Cu") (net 2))
 (segment (start 74.72045 83.82) (end 75.99055 82.5499) (width 0.1524) (layer "B.Cu") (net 12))
 (segment (start 78.53045 80.01) (end 79.80045 81.28) (width 0.1524) (layer "B.Cu") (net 12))
 (segment (start 75.99055 80.6449) (end 76.62545 80.01) (width 0.1524) (layer "B.Cu") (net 12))
 (segment (start 75.99055 82.5499) (end 75.99055 80.6449) (width 0.1524) (layer "B.Cu") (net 12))
 (segment (start 76.62545 80.01) (end 78.53045 80.01) (width 0.1524) (layer "B.Cu") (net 12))
 (segment (start 75.99045 97.79) (end 74.72045 99.06) (width 0.1524) (layer "B.Cu") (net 5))
 (segment (start 79.80045 99.06) (end 78.53045 97.79) (width 0.1524) (layer "B.Cu") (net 5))
 (segment (start 78.53045 97.79) (end 75.99045 97.79) (width 0.1524) (layer "B.Cu") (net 5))
 (segment (start 66.78295 86.36) (end 64.56045 86.36) (width 0.1524) (layer "B.Cu") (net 19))
 (segment (start 74.72045 91.44) (end 71.86295 91.44) (width 0.1524) (layer "B.Cu") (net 19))
 (segment (start 71.86295 91.44) (end 66.78295 86.36) (width 0.1524) (layer "B.Cu") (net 19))
 (segment (start 68.68795 83.82) (end 72.49795 87.63) (width 0.1524) (layer "B.Cu") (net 18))
 (segment (start 64.56045 83.82) (end 68.68795 83.82) (width 0.1524) (layer "B.Cu") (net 18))
 (segment (start 75.99045 87.63) (end 77.26045 88.9) (width 0.1524) (layer "B.Cu") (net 18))
 (segment (start 72.49795 87.63) (end 75.99045 87.63) (width 0.1524) (layer "B.Cu") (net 18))
 (segment (start 79.80045 96.52) (end 77.26045 96.52) (width 0.1524) (layer "B.Cu") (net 6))
 (segment (start 70.59295 111.76) (end 69.626371 110.793421) (width 0.1524) (layer "B.Cu") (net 32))
 (segment (start 74.72045 111.76) (end 70.59295 111.76) (width 0.1524) (layer "B.Cu") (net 32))
 (segment (start 69.626371 110.793421) (end 69.626371 106.668455) (width 0.1524) (layer "B.Cu") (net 32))
 (segment (start 66.14795 103.505) (end 65.83045 103.1875) (width 0.1524) (layer "F.Cu") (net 23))
 (segment (start 65.83045 97.79) (end 64.56045 96.52) (width 0.1524) (layer "F.Cu") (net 23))
 (segment (start 65.83045 103.1875) (end 65.83045 97.79) (width 0.1524) (layer "F.Cu") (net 23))
 (via (at 66.14795 103.505) (size 0.6096) (drill 0.3) (layers "F.Cu" "B.Cu") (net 23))
 (segment (start 74.08545 106.68) (end 74.72045 106.68) (width 0.1524) (layer "B.Cu") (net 23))
 (segment (start 66.46545 103.8225) (end 71.22795 103.8225) (width 0.1524) (layer "B.Cu") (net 23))
 (segment (start 71.22795 103.8225) (end 74.08545 106.68) (width 0.1524) (layer "B.Cu") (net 23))
 (segment (start 66.14795 103.505) (end 66.46545 103.8225) (width 0.1524) (layer "B.Cu") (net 23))
 (segment (start 79.80045 92.075) (end 79.80045 91.44) (width 0.1524) (layer "B.Cu") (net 8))
 (segment (start 77.26045 93.98) (end 77.89545 93.98) (width 0.1524) (layer "B.Cu") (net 8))
 (segment (start 77.89545 93.98) (end 79.80045 92.075) (width 0.1524) (layer "B.Cu") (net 8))
 (segment (start 75.99045 95.25) (end 74.72045 96.52) (width 0.1524) (layer "B.Cu") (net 7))
 (segment (start 78.53045 95.25) (end 75.99045 95.25) (width 0.1524) (layer "B.Cu") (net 7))
 (segment (start 79.80045 93.98) (end 78.53045 95.25) (width 0.1524) (layer "B.Cu") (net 7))
 (segment (start 65.83045 105.41) (end 64.56045 106.68) (width 0.1524) (layer "F.Cu") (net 27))
 (segment (start 66.14795 104.5591) (end 65.83045 104.8766) (width 0.1524) (layer "F.Cu") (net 27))
 (segment (start 65.83045 104.8766) (end 65.83045 105.41) (width 0.1524) (layer "F.Cu") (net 27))
 (via (at 66.14795 104.5591) (size 0.6096) (drill 0.3) (layers "F.Cu" "B.Cu") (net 27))
 (segment (start 66.14795 104.5591) (end 70.69455 104.5591) (width 0.1524) (layer "B.Cu") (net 27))
 (segment (start 74.08545 107.95) (end 75.99045 107.95) (width 0.1524) (layer "B.Cu") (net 27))
 (segment (start 70.69455 104.5591) (end 74.08545 107.95) (width 0.1524) (layer "B.Cu") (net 27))
 (segment (start 75.99045 107.95) (end 77.26045 109.22) (width 0.1524) (layer "B.Cu") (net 27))
 (segment (start 73.13295 111.91875) (end 74.2442 113.03) (width 0.4) (layer "F.Cu") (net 14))
 (segment (start 74.2442 113.03) (end 75.99045 113.03) (width 0.4) (layer "F.Cu") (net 14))
 (segment (start 75.99045 113.03) (end 77.26045 114.3) (width 0.4) (layer "F.Cu") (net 14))
 (segment (start 73.13295 80.3275) (end 73.13295 111.91875) (width 0.4) (layer "F.Cu") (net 14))
 (segment (start 74.72045 78.74) (end 73.13295 80.3275) (width 0.4) (layer "F.Cu") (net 14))
 (segment (start 79.80045 76.5175) (end 77.57795 78.74) (width 0.4) (layer "B.Cu") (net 14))
 (segment (start 77.57795 78.74) (end 77.260448 78.74) (width 0.4) (layer "B.Cu") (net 14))
 (segment (start 79.80045 76.2) (end 79.80045 76.5175) (width 0.6) (layer "B.Cu") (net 14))
 (segment (start 74.72045 78.74) (end 77.26045 78.74) (width 0.4) (layer "B.Cu") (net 14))
 (segment (start 77.26045 78.74) (end 77.260448 78.74) (width 0.6) (layer "B.Cu") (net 14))
 (segment (start 64.56045 109.22) (end 65.83045 107.95) (width 0.1524) (layer "F.Cu") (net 28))
 (segment (start 65.83045 106.3625) (end 67.100449 105.092501) (width 0.1524) (layer "F.Cu") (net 28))
 (segment (start 72.18045 114.3) (end 65.83045 114.3) (width 0.4) (layer "F.Cu") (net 28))
 (segment (start 65.83045 107.95) (end 65.83045 106.3625) (width 0.1524) (layer "F.Cu") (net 28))
 (segment (start 64.56045 113.03) (end 64.56045 109.22) (width 0.4) (layer "F.Cu") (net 28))
 (segment (start 65.83045 114.3) (end 64.56045 113.03) (width 0.4) (layer "F.Cu") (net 28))
 (segment (start 67.100449 105.092501) (end 67.100449 101.59212) (width 0.1524) (layer "F.Cu") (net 28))
 (segment (start 64.56045 81.28) (end 68.172013 84.891563) (width 0.1524) (layer "F.Cu") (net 17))
 (segment (start 68.172013 84.891563) (end 68.251387 84.891563) (width 0.1524) (layer "F.Cu") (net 17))
 (via (at 68.251387 84.891563) (size 0.6096) (drill 0.3) (layers "F.Cu" "B.Cu") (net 17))
 (segment (start 72.259825 88.9) (end 68.251387 84.891563) (width 0.1524) (layer "B.Cu") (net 17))
 (segment (start 74.72045 88.9) (end 72.259825 88.9) (width 0.1524) (layer "B.Cu") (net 17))
 (segment (start 68.37045 97.79) (end 64.56045 93.98) (width 0.1524) (layer "F.Cu") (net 22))
 (segment (start 71.22795 110.49) (end 68.37045 107.6325) (width 0.1524) (layer "F.Cu") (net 22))
 (segment (start 68.37045 107.6325) (end 68.37045 97.79) (width 0.1524) (layer "F.Cu") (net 22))
 (via (at 71.22795 110.49) (size 0.6096) (drill 0.3) (layers "F.Cu" "B.Cu") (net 22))
 (segment (start 75.99045 110.49) (end 77.26045 111.76) (width 0.1524) (layer "B.Cu") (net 22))
 (segment (start 71.22795 110.49) (end 75.99045 110.49) (width 0.1524) (layer "B.Cu") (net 22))
 (segment (start 74.5617 114.3) (end 74.72045 114.3) (width 0.4) (layer "F.Cu") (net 30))
 (segment (start 72.18045 111.91875) (end 74.5617 114.3) (width 0.4) (layer "F.Cu") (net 30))
 (segment (start 74.72045 76.2) (end 72.18045 78.74) (width 0.4) (layer "F.Cu") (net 30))
 (segment (start 72.18045 78.74) (end 72.18045 111.91875) (width 0.4) (layer "F.Cu") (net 30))
 (segment (start 68.37045 113.03) (end 78.53045 113.03) (width 0.1524) (layer "B.Cu") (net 33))
 (segment (start 67.100449 111.759999) (end 68.37045 113.03) (width 0.1524) (layer "B.Cu") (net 33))
 (segment (start 78.53045 113.03) (end 79.80045 114.3) (width 0.1524) (layer "B.Cu") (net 33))
 (segment (start 67.100449 106.67212) (end 67.100449 111.759999) (width 0.1524) (layer "B.Cu") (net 33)))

